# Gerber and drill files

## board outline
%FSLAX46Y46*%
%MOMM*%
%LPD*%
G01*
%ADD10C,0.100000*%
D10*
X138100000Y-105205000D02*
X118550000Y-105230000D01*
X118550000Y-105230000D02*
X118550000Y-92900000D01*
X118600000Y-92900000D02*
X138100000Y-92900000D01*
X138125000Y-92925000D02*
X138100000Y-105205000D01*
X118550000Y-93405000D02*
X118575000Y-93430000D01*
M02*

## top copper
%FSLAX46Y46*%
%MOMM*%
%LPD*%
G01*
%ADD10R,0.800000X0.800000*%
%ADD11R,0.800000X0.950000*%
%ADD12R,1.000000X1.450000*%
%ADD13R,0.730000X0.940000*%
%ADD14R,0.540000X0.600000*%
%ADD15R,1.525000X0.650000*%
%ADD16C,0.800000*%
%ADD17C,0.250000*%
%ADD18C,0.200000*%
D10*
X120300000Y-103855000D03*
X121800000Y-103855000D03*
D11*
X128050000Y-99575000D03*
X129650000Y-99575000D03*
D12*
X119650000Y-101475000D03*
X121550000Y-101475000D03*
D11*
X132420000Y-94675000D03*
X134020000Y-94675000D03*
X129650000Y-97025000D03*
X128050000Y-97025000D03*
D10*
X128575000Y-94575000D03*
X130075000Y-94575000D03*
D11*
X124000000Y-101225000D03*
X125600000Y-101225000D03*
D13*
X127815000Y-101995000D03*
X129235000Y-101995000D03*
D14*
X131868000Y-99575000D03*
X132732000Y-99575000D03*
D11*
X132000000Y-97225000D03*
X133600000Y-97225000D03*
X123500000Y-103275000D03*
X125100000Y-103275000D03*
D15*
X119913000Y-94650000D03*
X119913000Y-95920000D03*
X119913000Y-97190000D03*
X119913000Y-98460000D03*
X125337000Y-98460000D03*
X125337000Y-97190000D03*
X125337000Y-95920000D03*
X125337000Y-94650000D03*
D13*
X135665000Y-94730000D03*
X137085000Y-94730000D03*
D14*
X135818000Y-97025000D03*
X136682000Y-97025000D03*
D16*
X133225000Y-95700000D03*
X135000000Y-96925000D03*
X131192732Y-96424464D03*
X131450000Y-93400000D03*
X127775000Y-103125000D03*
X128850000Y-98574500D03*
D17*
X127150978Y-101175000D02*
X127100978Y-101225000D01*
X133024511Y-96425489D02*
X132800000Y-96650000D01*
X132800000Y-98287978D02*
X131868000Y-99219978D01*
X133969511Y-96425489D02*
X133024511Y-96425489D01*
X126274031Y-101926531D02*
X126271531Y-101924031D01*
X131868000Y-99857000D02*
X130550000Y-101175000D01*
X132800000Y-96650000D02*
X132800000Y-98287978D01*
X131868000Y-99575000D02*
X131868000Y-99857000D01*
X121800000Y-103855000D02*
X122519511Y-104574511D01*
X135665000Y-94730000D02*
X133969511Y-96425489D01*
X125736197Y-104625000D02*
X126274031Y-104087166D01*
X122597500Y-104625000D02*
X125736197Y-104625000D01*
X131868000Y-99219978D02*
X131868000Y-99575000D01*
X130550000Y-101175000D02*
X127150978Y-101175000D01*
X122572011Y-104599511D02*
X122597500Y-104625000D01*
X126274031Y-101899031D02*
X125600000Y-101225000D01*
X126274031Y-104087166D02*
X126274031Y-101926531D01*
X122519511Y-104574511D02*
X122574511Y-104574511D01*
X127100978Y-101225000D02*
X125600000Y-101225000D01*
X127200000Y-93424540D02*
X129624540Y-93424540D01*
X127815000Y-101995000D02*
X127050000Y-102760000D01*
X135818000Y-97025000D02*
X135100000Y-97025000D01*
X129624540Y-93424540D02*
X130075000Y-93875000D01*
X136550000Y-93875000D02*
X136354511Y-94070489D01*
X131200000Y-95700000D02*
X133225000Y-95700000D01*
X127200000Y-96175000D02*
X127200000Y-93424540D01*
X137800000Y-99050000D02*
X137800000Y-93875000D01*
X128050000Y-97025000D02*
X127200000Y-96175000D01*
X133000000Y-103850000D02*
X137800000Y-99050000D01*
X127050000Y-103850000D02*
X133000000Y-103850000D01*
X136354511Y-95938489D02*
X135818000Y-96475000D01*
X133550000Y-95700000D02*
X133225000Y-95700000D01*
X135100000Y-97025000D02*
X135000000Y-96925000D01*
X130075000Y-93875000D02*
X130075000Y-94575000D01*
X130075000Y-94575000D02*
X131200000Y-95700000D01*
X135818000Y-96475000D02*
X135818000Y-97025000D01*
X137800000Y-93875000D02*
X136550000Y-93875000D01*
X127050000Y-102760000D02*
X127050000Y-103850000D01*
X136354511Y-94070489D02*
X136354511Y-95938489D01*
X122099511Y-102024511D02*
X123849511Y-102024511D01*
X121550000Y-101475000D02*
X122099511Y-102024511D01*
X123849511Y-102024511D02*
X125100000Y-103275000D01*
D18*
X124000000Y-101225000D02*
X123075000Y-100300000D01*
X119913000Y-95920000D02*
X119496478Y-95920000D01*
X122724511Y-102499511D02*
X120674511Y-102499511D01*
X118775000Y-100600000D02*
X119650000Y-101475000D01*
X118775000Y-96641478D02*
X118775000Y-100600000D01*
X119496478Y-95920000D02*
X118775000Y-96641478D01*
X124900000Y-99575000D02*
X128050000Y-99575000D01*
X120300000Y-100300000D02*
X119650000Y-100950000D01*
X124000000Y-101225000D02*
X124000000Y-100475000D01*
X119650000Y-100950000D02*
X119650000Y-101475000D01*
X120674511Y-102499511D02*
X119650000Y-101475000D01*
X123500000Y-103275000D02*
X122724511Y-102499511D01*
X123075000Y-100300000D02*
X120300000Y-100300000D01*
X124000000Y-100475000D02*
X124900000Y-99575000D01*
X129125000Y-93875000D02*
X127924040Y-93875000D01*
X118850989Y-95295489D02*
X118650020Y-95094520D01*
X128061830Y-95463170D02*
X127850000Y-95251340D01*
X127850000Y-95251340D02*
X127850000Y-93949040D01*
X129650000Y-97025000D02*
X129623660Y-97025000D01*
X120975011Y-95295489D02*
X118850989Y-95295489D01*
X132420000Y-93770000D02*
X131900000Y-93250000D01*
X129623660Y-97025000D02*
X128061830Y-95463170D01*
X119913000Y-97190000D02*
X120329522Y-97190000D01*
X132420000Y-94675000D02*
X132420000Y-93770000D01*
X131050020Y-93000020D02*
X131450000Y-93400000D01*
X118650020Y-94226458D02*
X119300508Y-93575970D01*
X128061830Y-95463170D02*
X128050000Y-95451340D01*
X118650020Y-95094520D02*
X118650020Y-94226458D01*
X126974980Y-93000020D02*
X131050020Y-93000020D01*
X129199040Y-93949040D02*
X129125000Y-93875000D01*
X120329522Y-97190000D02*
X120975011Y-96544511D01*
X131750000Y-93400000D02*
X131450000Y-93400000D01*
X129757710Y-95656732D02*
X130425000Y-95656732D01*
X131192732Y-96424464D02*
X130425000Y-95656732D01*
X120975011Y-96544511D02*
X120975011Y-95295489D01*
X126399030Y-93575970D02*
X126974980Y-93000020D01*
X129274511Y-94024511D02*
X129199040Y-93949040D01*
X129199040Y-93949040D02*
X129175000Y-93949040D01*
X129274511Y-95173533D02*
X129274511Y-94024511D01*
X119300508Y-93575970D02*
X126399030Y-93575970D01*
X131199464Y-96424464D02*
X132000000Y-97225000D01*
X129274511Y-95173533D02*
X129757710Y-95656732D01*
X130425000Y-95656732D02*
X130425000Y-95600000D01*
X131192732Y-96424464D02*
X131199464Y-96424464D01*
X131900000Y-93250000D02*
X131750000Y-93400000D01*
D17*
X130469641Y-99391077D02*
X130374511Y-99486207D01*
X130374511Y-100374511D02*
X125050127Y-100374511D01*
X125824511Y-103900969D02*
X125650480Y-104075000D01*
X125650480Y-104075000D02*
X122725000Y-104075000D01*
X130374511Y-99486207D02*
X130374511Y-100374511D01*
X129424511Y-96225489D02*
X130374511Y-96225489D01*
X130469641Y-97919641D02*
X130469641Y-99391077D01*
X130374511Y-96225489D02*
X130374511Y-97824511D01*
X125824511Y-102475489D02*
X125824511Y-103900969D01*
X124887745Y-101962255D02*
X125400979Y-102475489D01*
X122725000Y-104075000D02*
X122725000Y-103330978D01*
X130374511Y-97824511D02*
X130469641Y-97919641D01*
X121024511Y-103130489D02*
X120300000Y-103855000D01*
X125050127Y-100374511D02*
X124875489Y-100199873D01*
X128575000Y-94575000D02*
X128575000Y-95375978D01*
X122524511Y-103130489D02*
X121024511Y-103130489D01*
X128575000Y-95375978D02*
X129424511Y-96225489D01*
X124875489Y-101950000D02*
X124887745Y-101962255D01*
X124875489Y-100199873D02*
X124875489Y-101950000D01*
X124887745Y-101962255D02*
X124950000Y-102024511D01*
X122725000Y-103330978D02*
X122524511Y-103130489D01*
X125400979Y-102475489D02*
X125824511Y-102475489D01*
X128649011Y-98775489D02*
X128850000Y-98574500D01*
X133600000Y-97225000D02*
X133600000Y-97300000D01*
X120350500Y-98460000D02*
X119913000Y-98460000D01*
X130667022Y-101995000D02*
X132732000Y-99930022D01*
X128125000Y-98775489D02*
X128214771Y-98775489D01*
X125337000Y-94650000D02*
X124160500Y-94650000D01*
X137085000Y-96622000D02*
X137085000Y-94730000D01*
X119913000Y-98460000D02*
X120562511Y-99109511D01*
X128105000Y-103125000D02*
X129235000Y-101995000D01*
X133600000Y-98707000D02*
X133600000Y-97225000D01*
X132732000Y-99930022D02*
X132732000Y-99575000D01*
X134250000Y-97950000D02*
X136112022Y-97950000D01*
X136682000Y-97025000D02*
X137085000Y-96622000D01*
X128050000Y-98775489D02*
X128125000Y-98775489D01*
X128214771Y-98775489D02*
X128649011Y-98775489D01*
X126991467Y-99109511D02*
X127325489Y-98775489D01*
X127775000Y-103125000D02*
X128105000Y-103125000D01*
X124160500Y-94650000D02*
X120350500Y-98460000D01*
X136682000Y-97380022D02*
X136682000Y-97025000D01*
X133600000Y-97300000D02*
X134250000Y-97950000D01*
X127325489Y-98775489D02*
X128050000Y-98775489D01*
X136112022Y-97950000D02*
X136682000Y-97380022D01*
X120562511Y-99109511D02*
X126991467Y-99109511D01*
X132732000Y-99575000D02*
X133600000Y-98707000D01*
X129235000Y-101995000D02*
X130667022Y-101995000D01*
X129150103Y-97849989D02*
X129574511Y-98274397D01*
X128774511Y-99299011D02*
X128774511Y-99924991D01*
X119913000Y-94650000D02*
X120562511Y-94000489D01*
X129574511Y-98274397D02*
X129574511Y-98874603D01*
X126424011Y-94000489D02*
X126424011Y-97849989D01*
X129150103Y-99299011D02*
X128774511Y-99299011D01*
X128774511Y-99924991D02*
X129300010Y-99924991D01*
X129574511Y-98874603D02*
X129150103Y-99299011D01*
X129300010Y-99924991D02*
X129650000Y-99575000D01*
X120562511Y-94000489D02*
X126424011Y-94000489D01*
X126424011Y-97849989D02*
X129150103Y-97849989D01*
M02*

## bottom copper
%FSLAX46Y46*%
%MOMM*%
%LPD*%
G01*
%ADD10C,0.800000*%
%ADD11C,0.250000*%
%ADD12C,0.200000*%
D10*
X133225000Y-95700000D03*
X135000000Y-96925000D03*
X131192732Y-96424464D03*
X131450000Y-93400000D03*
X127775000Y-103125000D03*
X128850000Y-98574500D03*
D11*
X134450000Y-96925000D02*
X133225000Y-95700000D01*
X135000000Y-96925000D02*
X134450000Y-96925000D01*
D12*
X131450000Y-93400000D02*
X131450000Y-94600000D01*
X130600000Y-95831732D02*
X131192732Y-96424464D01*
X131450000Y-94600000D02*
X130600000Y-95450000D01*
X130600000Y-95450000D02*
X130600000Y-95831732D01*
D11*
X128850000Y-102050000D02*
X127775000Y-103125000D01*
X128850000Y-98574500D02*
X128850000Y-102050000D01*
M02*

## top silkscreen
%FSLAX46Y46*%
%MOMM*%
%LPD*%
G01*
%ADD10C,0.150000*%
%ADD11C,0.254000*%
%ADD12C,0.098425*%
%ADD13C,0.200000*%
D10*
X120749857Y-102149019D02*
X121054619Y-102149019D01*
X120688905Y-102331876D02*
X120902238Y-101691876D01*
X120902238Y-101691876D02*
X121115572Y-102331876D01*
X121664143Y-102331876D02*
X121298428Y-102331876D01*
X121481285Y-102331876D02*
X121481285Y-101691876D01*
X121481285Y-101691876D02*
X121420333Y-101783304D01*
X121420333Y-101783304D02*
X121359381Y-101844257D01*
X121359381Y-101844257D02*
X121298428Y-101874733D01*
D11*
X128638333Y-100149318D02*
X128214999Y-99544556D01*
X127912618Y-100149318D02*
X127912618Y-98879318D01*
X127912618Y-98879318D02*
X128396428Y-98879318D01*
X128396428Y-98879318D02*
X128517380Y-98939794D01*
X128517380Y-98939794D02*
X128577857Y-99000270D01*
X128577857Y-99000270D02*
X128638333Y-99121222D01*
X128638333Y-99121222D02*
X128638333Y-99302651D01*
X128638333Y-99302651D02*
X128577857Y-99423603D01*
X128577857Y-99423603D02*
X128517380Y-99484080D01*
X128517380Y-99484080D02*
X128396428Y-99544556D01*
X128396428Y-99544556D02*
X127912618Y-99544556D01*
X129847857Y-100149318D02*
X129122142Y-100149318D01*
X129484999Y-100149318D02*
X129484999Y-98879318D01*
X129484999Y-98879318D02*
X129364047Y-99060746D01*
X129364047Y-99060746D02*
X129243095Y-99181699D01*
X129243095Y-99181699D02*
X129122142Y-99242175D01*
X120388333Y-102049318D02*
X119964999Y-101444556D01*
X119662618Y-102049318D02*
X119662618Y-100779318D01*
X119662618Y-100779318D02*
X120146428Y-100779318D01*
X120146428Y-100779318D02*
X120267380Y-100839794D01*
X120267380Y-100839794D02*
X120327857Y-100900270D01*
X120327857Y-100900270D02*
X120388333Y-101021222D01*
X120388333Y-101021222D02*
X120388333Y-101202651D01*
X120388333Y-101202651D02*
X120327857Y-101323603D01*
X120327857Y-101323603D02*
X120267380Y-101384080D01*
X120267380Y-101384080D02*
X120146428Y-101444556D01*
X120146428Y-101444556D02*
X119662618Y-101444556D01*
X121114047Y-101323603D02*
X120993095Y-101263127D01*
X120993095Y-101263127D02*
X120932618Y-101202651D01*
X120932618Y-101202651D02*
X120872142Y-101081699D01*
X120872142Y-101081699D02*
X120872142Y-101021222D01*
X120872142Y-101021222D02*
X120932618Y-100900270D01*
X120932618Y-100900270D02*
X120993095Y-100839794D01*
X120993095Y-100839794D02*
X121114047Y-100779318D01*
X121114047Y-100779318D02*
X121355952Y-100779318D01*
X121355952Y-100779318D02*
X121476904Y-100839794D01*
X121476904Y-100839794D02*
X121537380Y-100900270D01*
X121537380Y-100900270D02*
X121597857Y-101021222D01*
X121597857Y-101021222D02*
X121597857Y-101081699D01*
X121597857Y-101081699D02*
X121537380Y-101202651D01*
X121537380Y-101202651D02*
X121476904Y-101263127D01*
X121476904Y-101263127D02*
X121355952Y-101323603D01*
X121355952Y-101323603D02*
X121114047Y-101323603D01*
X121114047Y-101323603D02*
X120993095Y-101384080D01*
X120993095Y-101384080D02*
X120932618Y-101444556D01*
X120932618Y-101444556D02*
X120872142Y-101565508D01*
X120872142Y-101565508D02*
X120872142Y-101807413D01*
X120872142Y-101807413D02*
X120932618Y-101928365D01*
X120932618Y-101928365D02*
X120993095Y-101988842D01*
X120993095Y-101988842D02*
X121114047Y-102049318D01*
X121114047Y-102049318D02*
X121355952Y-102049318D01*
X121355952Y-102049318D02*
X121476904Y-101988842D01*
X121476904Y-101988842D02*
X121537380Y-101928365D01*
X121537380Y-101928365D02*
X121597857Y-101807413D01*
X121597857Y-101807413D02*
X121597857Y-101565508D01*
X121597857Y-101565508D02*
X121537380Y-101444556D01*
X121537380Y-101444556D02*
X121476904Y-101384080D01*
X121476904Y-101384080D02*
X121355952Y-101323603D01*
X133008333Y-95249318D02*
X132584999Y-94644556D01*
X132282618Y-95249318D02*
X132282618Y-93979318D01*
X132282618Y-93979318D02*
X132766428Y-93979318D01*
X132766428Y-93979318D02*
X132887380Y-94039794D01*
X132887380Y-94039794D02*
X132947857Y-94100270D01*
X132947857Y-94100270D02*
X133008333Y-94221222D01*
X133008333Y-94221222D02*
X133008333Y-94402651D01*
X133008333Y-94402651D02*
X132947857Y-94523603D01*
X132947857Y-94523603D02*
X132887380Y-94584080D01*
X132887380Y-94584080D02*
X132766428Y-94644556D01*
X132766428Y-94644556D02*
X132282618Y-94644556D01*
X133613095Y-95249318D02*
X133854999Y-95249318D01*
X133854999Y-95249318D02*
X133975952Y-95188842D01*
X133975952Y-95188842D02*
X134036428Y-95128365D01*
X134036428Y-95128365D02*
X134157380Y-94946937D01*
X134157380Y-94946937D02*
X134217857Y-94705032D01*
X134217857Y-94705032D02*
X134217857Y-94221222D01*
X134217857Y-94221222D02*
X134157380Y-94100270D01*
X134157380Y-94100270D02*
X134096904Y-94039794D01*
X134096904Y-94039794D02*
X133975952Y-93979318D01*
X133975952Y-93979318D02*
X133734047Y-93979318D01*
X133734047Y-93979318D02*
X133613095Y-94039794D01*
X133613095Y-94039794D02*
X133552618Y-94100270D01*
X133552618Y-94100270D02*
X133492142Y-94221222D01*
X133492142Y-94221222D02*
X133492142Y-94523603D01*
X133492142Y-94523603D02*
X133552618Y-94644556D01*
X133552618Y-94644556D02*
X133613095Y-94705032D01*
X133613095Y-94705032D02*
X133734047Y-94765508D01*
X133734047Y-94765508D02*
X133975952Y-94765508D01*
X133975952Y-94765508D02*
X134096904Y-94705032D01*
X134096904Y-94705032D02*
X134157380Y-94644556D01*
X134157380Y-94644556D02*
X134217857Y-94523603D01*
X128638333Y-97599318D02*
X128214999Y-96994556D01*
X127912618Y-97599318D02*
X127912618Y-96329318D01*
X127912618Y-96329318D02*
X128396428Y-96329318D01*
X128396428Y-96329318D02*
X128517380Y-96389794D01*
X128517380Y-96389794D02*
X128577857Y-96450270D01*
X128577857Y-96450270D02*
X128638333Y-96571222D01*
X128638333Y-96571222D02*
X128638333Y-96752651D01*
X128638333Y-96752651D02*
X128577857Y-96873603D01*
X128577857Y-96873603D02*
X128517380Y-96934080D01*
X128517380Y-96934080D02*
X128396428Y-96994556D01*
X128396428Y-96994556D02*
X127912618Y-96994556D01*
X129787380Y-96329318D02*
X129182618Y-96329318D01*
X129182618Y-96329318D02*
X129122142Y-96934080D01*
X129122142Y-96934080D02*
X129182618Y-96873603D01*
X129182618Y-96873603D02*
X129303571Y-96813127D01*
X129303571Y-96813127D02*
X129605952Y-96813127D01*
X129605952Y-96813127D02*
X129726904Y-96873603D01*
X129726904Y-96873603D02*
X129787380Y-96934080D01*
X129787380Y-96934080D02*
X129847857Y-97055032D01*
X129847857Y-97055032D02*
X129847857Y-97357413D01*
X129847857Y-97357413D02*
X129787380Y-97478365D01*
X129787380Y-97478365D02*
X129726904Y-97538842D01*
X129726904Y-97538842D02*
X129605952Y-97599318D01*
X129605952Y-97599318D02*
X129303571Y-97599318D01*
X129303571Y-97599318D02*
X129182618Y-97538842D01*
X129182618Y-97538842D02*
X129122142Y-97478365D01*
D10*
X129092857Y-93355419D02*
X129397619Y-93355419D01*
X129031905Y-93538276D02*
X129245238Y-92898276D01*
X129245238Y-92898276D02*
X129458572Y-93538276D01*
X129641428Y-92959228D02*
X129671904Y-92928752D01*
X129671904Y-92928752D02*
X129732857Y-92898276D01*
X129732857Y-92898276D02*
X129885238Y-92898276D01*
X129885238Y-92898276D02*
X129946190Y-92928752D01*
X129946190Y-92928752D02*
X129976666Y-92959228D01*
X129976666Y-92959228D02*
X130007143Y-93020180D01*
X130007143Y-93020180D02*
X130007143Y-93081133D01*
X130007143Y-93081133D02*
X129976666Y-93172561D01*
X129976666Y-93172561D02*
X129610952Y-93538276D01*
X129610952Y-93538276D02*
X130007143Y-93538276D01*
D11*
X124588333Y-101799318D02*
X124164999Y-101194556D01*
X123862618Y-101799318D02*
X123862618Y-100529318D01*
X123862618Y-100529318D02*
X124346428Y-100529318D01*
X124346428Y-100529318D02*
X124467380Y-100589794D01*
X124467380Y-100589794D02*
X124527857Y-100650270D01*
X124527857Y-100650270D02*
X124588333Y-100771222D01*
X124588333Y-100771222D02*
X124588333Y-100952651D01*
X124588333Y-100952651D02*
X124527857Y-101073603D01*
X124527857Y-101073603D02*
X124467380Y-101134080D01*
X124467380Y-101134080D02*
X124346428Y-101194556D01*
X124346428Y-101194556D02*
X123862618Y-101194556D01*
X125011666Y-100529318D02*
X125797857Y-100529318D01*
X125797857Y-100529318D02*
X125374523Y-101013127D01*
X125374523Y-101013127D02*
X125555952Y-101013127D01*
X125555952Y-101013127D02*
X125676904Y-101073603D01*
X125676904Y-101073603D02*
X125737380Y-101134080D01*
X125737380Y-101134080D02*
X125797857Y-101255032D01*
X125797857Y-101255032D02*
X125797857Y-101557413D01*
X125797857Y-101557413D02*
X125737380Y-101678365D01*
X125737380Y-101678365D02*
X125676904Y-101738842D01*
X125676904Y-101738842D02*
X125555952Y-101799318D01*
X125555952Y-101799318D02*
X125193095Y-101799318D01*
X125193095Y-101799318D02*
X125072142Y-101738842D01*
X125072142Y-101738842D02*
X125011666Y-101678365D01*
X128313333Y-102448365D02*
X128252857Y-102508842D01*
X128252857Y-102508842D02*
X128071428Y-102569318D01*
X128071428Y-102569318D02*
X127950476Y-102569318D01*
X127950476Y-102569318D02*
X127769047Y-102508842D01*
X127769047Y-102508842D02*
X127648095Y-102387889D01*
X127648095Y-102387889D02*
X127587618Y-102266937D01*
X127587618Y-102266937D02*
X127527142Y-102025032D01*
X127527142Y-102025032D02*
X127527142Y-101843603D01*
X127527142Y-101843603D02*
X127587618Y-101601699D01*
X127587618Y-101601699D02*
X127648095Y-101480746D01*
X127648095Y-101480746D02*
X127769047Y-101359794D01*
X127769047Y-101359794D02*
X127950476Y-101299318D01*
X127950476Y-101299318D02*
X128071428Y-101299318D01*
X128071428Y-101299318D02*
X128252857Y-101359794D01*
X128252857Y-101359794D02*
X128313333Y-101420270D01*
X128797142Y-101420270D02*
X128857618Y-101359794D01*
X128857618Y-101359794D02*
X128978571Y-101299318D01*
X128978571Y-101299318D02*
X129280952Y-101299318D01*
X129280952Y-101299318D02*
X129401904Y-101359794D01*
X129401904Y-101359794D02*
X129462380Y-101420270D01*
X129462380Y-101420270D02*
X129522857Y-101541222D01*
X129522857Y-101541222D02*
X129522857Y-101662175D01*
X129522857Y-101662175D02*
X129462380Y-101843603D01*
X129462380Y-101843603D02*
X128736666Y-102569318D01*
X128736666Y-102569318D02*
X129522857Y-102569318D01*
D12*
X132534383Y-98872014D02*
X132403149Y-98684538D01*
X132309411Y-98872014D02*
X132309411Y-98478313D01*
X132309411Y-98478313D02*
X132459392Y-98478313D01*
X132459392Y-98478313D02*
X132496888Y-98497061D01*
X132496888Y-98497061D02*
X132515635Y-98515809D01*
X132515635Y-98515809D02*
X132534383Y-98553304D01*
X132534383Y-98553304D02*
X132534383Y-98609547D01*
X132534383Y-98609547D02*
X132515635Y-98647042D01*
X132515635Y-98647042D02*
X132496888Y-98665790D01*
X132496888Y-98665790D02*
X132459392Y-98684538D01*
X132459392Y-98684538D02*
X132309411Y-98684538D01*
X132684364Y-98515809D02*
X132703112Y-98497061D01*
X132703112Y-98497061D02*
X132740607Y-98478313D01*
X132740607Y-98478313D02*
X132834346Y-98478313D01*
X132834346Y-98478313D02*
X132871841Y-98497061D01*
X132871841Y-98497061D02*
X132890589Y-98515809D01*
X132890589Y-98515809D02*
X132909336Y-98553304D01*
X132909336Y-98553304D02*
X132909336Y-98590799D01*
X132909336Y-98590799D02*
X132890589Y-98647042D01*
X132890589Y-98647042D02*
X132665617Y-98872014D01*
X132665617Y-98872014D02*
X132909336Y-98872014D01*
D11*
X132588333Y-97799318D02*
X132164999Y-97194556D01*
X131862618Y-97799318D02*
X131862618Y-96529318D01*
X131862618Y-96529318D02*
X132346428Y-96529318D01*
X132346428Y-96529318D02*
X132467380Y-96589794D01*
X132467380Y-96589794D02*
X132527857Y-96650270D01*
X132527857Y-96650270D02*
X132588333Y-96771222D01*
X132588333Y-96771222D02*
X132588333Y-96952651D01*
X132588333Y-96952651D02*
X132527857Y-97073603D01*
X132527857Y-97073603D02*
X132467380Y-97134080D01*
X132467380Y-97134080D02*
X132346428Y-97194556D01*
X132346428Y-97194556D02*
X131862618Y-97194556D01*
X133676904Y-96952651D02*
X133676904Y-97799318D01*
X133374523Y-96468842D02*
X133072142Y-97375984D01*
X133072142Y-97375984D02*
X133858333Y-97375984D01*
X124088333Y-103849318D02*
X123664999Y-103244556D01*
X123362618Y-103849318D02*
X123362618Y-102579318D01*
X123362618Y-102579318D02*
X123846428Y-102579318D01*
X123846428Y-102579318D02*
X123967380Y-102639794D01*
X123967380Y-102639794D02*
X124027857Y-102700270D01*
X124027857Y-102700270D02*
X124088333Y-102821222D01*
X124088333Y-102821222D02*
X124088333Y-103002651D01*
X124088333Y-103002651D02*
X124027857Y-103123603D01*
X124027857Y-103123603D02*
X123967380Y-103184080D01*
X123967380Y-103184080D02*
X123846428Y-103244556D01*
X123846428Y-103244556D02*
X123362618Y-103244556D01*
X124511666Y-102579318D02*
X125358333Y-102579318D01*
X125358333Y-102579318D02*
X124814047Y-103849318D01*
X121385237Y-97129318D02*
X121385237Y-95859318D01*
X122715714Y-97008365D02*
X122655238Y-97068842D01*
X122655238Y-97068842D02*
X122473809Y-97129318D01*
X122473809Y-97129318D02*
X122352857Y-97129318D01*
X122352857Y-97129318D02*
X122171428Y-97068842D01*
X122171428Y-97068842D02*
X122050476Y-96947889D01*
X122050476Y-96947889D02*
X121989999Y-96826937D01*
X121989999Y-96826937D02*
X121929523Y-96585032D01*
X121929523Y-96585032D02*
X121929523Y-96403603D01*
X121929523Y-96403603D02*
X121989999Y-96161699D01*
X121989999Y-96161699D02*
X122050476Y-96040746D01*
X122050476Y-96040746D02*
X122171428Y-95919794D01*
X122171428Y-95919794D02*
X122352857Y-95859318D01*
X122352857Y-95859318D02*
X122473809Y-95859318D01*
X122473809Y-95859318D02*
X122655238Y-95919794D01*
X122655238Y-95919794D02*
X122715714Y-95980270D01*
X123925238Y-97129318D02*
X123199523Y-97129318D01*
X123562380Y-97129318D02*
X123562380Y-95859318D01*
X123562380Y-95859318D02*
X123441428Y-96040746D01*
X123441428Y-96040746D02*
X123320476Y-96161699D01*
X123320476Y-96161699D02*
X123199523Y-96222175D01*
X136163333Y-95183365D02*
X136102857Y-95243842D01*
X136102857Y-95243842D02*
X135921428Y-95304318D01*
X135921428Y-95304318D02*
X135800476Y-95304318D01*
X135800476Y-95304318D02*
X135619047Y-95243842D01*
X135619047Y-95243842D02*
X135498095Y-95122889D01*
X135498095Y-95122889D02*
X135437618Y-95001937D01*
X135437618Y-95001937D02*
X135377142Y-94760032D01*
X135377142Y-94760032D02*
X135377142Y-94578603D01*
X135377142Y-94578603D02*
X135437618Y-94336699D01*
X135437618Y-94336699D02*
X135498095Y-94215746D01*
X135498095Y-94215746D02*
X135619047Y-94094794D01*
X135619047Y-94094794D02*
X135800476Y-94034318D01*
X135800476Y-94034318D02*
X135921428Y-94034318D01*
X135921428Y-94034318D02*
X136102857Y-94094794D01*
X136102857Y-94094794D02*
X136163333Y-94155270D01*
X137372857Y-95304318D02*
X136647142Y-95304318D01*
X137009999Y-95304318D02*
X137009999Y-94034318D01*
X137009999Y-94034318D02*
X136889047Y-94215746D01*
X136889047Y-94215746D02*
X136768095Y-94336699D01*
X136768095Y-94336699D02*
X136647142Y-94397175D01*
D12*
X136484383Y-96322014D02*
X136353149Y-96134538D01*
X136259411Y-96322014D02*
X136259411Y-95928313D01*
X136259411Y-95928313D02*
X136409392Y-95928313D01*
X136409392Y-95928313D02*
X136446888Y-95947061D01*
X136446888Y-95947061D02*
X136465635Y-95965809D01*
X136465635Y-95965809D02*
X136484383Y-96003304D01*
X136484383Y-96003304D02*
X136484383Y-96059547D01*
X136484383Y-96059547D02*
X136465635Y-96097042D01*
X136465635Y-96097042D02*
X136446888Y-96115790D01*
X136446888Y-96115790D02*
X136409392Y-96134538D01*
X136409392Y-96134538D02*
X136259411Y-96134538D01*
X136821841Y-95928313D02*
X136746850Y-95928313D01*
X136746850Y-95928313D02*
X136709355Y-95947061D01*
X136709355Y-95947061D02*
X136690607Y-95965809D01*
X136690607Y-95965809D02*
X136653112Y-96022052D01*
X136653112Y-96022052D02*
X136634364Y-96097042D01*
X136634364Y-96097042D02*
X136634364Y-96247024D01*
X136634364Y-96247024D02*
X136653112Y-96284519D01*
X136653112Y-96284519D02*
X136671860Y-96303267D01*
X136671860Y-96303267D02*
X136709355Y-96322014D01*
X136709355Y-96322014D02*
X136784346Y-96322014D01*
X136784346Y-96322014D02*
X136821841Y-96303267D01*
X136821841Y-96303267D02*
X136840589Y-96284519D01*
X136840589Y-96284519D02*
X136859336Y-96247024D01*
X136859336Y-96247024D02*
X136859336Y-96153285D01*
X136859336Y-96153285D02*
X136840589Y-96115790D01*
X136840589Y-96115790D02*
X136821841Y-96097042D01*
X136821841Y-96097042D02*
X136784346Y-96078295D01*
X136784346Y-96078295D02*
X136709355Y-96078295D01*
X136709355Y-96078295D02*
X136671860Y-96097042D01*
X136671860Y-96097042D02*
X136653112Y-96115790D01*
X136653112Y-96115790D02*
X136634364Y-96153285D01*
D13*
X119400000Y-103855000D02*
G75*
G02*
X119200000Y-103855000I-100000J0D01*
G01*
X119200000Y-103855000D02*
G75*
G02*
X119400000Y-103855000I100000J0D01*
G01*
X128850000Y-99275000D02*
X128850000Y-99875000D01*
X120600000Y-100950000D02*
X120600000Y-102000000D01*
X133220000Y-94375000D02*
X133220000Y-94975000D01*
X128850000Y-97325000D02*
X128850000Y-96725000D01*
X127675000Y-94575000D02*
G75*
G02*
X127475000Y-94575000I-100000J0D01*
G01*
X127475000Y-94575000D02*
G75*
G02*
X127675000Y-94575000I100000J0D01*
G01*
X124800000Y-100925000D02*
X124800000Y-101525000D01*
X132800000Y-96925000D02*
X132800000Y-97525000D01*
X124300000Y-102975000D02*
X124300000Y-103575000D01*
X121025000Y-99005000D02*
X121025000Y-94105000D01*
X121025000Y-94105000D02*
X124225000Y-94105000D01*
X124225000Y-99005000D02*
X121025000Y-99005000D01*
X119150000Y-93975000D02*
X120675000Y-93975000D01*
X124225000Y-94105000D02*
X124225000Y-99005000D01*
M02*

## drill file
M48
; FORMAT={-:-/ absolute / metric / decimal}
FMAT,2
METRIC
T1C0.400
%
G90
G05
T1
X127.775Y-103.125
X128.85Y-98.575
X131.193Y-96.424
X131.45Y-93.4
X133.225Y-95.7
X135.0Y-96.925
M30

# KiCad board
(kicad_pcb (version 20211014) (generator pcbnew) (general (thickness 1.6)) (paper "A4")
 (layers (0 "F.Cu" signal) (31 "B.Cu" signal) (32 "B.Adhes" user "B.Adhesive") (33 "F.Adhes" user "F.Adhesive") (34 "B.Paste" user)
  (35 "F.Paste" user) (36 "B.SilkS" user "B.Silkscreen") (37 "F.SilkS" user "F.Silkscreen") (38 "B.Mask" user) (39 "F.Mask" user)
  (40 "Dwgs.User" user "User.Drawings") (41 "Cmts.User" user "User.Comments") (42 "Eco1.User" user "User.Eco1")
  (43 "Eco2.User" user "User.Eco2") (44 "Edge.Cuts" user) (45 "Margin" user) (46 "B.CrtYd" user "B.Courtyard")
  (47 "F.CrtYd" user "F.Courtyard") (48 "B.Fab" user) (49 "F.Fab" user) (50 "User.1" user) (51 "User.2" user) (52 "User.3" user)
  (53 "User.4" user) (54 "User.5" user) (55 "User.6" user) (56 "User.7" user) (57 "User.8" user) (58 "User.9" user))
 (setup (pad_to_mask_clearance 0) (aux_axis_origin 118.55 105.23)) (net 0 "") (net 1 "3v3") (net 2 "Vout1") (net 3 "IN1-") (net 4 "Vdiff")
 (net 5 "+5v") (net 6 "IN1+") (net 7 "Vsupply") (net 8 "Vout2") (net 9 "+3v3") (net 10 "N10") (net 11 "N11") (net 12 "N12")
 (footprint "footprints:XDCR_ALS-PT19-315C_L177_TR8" (layer "F.Cu") (at 121.05 103.855)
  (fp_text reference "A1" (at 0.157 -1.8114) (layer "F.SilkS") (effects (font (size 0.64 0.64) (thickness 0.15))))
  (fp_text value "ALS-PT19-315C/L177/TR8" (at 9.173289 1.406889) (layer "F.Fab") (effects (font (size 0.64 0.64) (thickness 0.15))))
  (fp_circle (center -1.75 0) (end -1.65 0) (layer "F.SilkS") (width 0.2) (fill none))
  (pad "1" smd rect locked (at -0.75 0) (size 0.8 0.8) (layers "F.Cu" "F.Paste" "F.Mask") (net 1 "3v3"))
  (pad "2" smd rect locked (at 0.75 0) (size 0.8 0.8) (layers "F.Cu" "F.Paste" "F.Mask") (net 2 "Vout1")))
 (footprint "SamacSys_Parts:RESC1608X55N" (layer "F.Cu") (at 128.85 99.575)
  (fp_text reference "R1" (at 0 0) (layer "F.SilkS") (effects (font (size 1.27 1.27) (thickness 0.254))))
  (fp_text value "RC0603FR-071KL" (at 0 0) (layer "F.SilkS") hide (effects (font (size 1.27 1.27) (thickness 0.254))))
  (fp_line (start 0 -0.3) (end 0 0.3) (layer "F.SilkS") (width 0.2))
  (pad "1" smd rect locked (at -0.8 0) (size 0.8 0.95) (layers "F.Cu" "F.Paste" "F.Mask") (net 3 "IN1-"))
  (pad "2" smd rect locked (at 0.8 0) (size 0.8 0.95) (layers "F.Cu" "F.Paste" "F.Mask") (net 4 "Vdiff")))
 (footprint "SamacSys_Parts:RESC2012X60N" (layer "F.Cu") (at 120.6 101.475)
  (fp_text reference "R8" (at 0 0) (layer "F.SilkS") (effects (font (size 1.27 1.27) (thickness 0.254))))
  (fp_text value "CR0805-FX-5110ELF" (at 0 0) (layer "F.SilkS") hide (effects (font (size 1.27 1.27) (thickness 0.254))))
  (fp_line (start 0 -0.525) (end 0 0.525) (layer "F.SilkS") (width 0.2))
  (pad "1" smd rect locked (at -0.95 0) (size 1 1.45) (layers "F.Cu" "F.Paste" "F.Mask") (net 3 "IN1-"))
  (pad "2" smd rect locked (at 0.95 0) (size 1 1.45) (layers "F.Cu" "F.Paste" "F.Mask") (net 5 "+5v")))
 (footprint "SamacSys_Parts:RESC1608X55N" (layer "F.Cu") (at 133.22 94.675)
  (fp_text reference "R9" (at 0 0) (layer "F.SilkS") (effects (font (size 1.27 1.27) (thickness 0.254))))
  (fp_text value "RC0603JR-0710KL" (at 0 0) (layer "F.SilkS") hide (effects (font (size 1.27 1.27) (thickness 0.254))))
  (fp_line (start 0 -0.3) (end 0 0.3) (layer "F.SilkS") (width 0.2))
  (pad "1" smd rect locked (at -0.8 0) (size 0.8 0.95) (layers "F.Cu" "F.Paste" "F.Mask") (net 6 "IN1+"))
  (pad "2" smd rect locked (at 0.8 0) (size 0.8 0.95) (layers "F.Cu" "F.Paste" "F.Mask") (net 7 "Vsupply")))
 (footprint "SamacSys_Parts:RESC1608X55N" (layer "F.Cu") (at 128.85 97.025 180)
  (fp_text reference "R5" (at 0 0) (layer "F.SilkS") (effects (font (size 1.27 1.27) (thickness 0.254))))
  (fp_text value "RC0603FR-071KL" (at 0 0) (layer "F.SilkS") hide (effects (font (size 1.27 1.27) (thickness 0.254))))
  (fp_line (start 0 -0.3) (end 0 0.3) (layer "F.SilkS") (width 0.2))
  (pad "1" smd rect locked (at -0.8 0 180) (size 0.8 0.95) (layers "F.Cu" "F.Paste" "F.Mask") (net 6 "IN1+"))
  (pad "2" smd rect locked (at 0.8 0 180) (size 0.8 0.95) (layers "F.Cu" "F.Paste" "F.Mask") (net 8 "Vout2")))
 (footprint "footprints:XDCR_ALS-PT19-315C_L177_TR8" (layer "F.Cu") (at 129.325 94.575)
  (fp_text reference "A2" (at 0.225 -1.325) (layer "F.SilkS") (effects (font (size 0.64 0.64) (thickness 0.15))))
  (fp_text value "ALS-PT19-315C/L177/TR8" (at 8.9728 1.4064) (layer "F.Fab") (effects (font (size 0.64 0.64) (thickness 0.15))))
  (fp_circle (center -1.75 0) (end -1.65 0) (layer "F.SilkS") (width 0.2) (fill none))
  (pad "1" smd rect locked (at -0.75 0) (size 0.8 0.8) (layers "F.Cu" "F.Paste" "F.Mask") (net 1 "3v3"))
  (pad "2" smd rect locked (at 0.75 0) (size 0.8 0.8) (layers "F.Cu" "F.Paste" "F.Mask") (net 8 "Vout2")))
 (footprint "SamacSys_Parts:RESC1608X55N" (layer "F.Cu") (at 124.8 101.225)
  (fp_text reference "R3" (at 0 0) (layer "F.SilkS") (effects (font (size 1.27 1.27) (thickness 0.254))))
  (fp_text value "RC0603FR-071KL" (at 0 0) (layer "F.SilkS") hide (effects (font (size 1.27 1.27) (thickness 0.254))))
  (fp_line (start 0 -0.3) (end 0 0.3) (layer "F.SilkS") (width 0.2))
  (pad "1" smd rect locked (at -0.8 0) (size 0.8 0.95) (layers "F.Cu" "F.Paste" "F.Mask") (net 3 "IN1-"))
  (pad "2" smd rect locked (at 0.8 0) (size 0.8 0.95) (layers "F.Cu" "F.Paste" "F.Mask") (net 2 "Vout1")))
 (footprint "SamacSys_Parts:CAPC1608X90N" (layer "F.Cu") (at 128.525 101.995)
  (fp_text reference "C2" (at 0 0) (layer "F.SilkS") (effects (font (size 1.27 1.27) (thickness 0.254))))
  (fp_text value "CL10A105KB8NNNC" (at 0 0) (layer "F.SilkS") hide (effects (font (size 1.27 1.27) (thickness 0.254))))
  (pad "1" smd rect locked (at -0.71 0) (size 0.73 0.94) (layers "F.Cu" "F.Paste" "F.Mask") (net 8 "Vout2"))
  (pad "2" smd rect locked (at 0.71 0) (size 0.73 0.94) (layers "F.Cu" "F.Paste" "F.Mask") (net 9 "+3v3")))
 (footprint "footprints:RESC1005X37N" (layer "F.Cu") (at 132.3 99.575)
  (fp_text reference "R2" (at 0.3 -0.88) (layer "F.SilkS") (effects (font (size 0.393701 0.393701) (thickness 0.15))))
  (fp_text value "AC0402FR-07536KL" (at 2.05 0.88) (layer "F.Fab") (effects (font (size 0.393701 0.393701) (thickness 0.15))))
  (pad "1" smd rect locked (at -0.432 0) (size 0.54 0.6) (layers "F.Cu" "F.Paste" "F.Mask") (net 2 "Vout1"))
  (pad "2" smd rect locked (at 0.432 0) (size 0.54 0.6) (layers "F.Cu" "F.Paste" "F.Mask") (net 9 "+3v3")))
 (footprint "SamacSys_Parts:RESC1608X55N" (layer "F.Cu") (at 132.8 97.225)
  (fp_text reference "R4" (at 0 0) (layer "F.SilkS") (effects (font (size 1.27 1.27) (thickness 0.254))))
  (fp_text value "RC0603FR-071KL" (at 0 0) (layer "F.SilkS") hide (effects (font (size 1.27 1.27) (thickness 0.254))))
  (fp_line (start 0 -0.3) (end 0 0.3) (layer "F.SilkS") (width 0.2))
  (pad "1" smd rect locked (at -0.8 0) (size 0.8 0.95) (layers "F.Cu" "F.Paste" "F.Mask") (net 6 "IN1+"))
  (pad "2" smd rect locked (at 0.8 0) (size 0.8 0.95) (layers "F.Cu" "F.Paste" "F.Mask") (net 9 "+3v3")))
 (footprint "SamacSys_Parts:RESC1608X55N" (layer "F.Cu") (at 124.3 103.275)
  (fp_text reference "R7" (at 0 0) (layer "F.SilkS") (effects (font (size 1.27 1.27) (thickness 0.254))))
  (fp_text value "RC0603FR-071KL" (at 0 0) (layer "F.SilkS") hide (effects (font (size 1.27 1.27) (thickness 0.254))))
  (fp_line (start 0 -0.3) (end 0 0.3) (layer "F.SilkS") (width 0.2))
  (pad "1" smd rect locked (at -0.8 0) (size 0.8 0.95) (layers "F.Cu" "F.Paste" "F.Mask") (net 3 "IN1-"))
  (pad "2" smd rect locked (at 0.8 0) (size 0.8 0.95) (layers "F.Cu" "F.Paste" "F.Mask") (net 5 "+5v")))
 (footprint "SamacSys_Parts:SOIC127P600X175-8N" (layer "F.Cu") (at 122.625 96.555)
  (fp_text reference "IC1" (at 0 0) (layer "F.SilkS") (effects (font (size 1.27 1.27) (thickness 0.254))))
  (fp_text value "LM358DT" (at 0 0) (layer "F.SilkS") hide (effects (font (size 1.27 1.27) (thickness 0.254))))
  (fp_line (start -1.6 2.45) (end -1.6 -2.45) (layer "F.SilkS") (width 0.2))
  (fp_line (start -1.6 -2.45) (end 1.6 -2.45) (layer "F.SilkS") (width 0.2))
  (fp_line (start 1.6 2.45) (end -1.6 2.45) (layer "F.SilkS") (width 0.2))
  (fp_line (start -3.475 -2.58) (end -1.95 -2.58) (layer "F.SilkS") (width 0.2))
  (fp_line (start 1.6 -2.45) (end 1.6 2.45) (layer "F.SilkS") (width 0.2))
  (pad "1" smd rect locked (at -2.712 -1.905 90) (size 0.65 1.525) (layers "F.Cu" "F.Paste" "F.Mask") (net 4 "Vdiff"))
  (pad "2" smd rect locked (at -2.712 -0.635 90) (size 0.65 1.525) (layers "F.Cu" "F.Paste" "F.Mask") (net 3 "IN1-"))
  (pad "3" smd rect locked (at -2.712 0.635 90) (size 0.65 1.525) (layers "F.Cu" "F.Paste" "F.Mask") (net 6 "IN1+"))
  (pad "4" smd rect locked (at -2.712 1.905 90) (size 0.65 1.525) (layers "F.Cu" "F.Paste" "F.Mask") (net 9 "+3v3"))
  (pad "5" smd rect locked (at 2.712 1.905 90) (size 0.65 1.525) (layers "F.Cu" "F.Paste" "F.Mask") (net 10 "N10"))
  (pad "6" smd rect locked (at 2.712 0.635 90) (size 0.65 1.525) (layers "F.Cu" "F.Paste" "F.Mask") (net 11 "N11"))
  (pad "7" smd rect locked (at 2.712 -0.635 90) (size 0.65 1.525) (layers "F.Cu" "F.Paste" "F.Mask") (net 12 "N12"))
  (pad "8" smd rect locked (at 2.712 -1.905 90) (size 0.65 1.525) (layers "F.Cu" "F.Paste" "F.Mask") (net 9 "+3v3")))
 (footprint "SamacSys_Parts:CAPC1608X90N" (layer "F.Cu") (at 136.375 94.73)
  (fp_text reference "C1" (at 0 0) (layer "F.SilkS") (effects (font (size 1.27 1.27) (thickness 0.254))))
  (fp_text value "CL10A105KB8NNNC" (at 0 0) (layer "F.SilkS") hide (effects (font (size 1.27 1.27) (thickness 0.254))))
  (pad "1" smd rect locked (at -0.71 0) (size 0.73 0.94) (layers "F.Cu" "F.Paste" "F.Mask") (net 2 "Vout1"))
  (pad "2" smd rect locked (at 0.71 0) (size 0.73 0.94) (layers "F.Cu" "F.Paste" "F.Mask") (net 9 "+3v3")))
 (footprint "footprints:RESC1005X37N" (layer "F.Cu") (at 136.25 97.025)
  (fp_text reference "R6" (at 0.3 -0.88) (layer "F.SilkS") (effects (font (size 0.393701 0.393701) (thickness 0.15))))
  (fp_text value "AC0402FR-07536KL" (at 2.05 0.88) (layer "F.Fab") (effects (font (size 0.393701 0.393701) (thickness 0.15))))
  (pad "1" smd rect locked (at -0.432 0) (size 0.54 0.6) (layers "F.Cu" "F.Paste" "F.Mask") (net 8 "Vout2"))
  (pad "2" smd rect locked (at 0.432 0) (size 0.54 0.6) (layers "F.Cu" "F.Paste" "F.Mask") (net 9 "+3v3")))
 (gr_line (start 138.1 105.205) (end 118.55 105.23) (layer "Edge.Cuts") (width 0.1))
 (gr_line (start 118.55 105.23) (end 118.55 92.9) (layer "Edge.Cuts") (width 0.1))
 (gr_line (start 118.6 92.9) (end 138.1 92.9) (layer "Edge.Cuts") (width 0.1))
 (gr_line (start 138.125 92.925) (end 138.1 105.205) (layer "Edge.Cuts") (width 0.1))
 (gr_line (start 118.55 93.405) (end 118.575 93.43) (layer "Edge.Cuts") (width 0.1))
 (segment (start 127.150978 101.175) (end 127.100978 101.225) (width 0.25) (layer "F.Cu") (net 2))
 (segment (start 133.024511 96.425489) (end 132.8 96.65) (width 0.25) (layer "F.Cu") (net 2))
 (segment (start 132.8 98.287978) (end 131.868 99.219978) (width 0.25) (layer "F.Cu") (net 2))
 (segment (start 133.969511 96.425489) (end 133.024511 96.425489) (width 0.25) (layer "F.Cu") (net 2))
 (segment (start 126.274031 101.926531) (end 126.271531 101.924031) (width 0.25) (layer "F.Cu") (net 2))
 (segment (start 131.868 99.857) (end 130.55 101.175) (width 0.25) (layer "F.Cu") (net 2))
 (segment (start 132.8 96.65) (end 132.8 98.287978) (width 0.25) (layer "F.Cu") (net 2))
 (segment (start 131.868 99.575) (end 131.868 99.857) (width 0.25) (layer "F.Cu") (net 2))
 (segment (start 121.8 103.855) (end 122.519511 104.574511) (width 0.25) (layer "F.Cu") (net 2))
 (segment (start 135.665 94.73) (end 133.969511 96.425489) (width 0.25) (layer "F.Cu") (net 2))
 (segment (start 125.736197 104.625) (end 126.274031 104.087166) (width 0.25) (layer "F.Cu") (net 2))
 (segment (start 122.5975 104.625) (end 125.736197 104.625) (width 0.25) (layer "F.Cu") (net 2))
 (segment (start 131.868 99.219978) (end 131.868 99.575) (width 0.25) (layer "F.Cu") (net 2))
 (segment (start 130.55 101.175) (end 127.150978 101.175) (width 0.25) (layer "F.Cu") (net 2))
 (segment (start 122.572011 104.599511) (end 122.5975 104.625) (width 0.25) (layer "F.Cu") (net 2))
 (segment (start 126.274031 101.899031) (end 125.6 101.225) (width 0.25) (layer "F.Cu") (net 2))
 (segment (start 126.274031 104.087166) (end 126.274031 101.926531) (width 0.25) (layer "F.Cu") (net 2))
 (segment (start 122.519511 104.574511) (end 122.574511 104.574511) (width 0.25) (layer "F.Cu") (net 2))
 (segment (start 127.100978 101.225) (end 125.6 101.225) (width 0.25) (layer "F.Cu") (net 2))
 (segment (start 127.2 93.42454) (end 129.62454 93.42454) (width 0.25) (layer "F.Cu") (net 8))
 (segment (start 127.815 101.995) (end 127.05 102.76) (width 0.25) (layer "F.Cu") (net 8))
 (segment (start 135.818 97.025) (end 135.1 97.025) (width 0.25) (layer "F.Cu") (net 8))
 (segment (start 129.62454 93.42454) (end 130.075 93.875) (width 0.25) (layer "F.Cu") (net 8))
 (segment (start 136.55 93.875) (end 136.354511 94.070489) (width 0.25) (layer "F.Cu") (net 8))
 (segment (start 131.2 95.7) (end 133.225 95.7) (width 0.25) (layer "F.Cu") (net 8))
 (segment (start 127.2 96.175) (end 127.2 93.42454) (width 0.25) (layer "F.Cu") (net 8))
 (segment (start 137.8 99.05) (end 137.8 93.875) (width 0.25) (layer "F.Cu") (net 8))
 (segment (start 128.05 97.025) (end 127.2 96.175) (width 0.25) (layer "F.Cu") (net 8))
 (segment (start 133 103.85) (end 137.8 99.05) (width 0.25) (layer "F.Cu") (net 8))
 (segment (start 127.05 103.85) (end 133 103.85) (width 0.25) (layer "F.Cu") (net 8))
 (segment (start 136.354511 95.938489) (end 135.818 96.475) (width 0.25) (layer "F.Cu") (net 8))
 (segment (start 133.55 95.7) (end 133.225 95.7) (width 0.25) (layer "F.Cu") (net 8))
 (segment (start 135.1 97.025) (end 135 96.925) (width 0.25) (layer "F.Cu") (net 8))
 (segment (start 130.075 93.875) (end 130.075 94.575) (width 0.25) (layer "F.Cu") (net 8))
 (segment (start 130.075 94.575) (end 131.2 95.7) (width 0.25) (layer "F.Cu") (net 8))
 (segment (start 135.818 96.475) (end 135.818 97.025) (width 0.25) (layer "F.Cu") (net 8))
 (segment (start 137.8 93.875) (end 136.55 93.875) (width 0.25) (layer "F.Cu") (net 8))
 (segment (start 127.05 102.76) (end 127.05 103.85) (width 0.25) (layer "F.Cu") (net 8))
 (segment (start 136.354511 94.070489) (end 136.354511 95.938489) (width 0.25) (layer "F.Cu") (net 8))
 (via (at 133.225 95.7) (size 0.8) (drill 0.4) (layers "F.Cu" "B.Cu") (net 8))
 (via (at 135 96.925) (size 0.8) (drill 0.4) (layers "F.Cu" "B.Cu") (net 8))
 (segment (start 134.45 96.925) (end 133.225 95.7) (width 0.25) (layer "B.Cu") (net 8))
 (segment (start 135 96.925) (end 134.45 96.925) (width 0.25) (layer "B.Cu") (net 8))
 (segment (start 122.099511 102.024511) (end 123.849511 102.024511) (width 0.25) (layer "F.Cu") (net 5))
 (segment (start 121.55 101.475) (end 122.099511 102.024511) (width 0.25) (layer "F.Cu") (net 5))
 (segment (start 123.849511 102.024511) (end 125.1 103.275) (width 0.25) (layer "F.Cu") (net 5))
 (segment (start 124 101.225) (end 123.075 100.3) (width 0.2) (layer "F.Cu") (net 3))
 (segment (start 119.913 95.92) (end 119.496478 95.92) (width 0.2) (layer "F.Cu") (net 3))
 (segment (start 122.724511 102.499511) (end 120.674511 102.499511) (width 0.2) (layer "F.Cu") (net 3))
 (segment (start 118.775 100.6) (end 119.65 101.475) (width 0.2) (layer "F.Cu") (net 3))
 (segment (start 118.775 96.641478) (end 118.775 100.6) (width 0.2) (layer "F.Cu") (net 3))
 (segment (start 119.496478 95.92) (end 118.775 96.641478) (width 0.2) (layer "F.Cu") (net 3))
 (segment (start 124.9 99.575) (end 128.05 99.575) (width 0.2) (layer "F.Cu") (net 3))
 (segment (start 120.3 100.3) (end 119.65 100.95) (width 0.2) (layer "F.Cu") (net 3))
 (segment (start 124 101.225) (end 124 100.475) (width 0.2) (layer "F.Cu") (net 3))
 (segment (start 119.65 100.95) (end 119.65 101.475) (width 0.2) (layer "F.Cu") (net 3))
 (segment (start 120.674511 102.499511) (end 119.65 101.475) (width 0.2) (layer "F.Cu") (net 3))
 (segment (start 123.5 103.275) (end 122.724511 102.499511) (width 0.2) (layer "F.Cu") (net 3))
 (segment (start 123.075 100.3) (end 120.3 100.3) (width 0.2) (layer "F.Cu") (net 3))
 (segment (start 124 100.475) (end 124.9 99.575) (width 0.2) (layer "F.Cu") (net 3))
 (segment (start 129.125 93.875) (end 127.92404 93.875) (width 0.2) (layer "F.Cu") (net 6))
 (segment (start 118.850989 95.295489) (end 118.65002 95.09452) (width 0.2) (layer "F.Cu") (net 6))
 (segment (start 128.06183 95.46317) (end 127.85 95.25134) (width 0.2) (layer "F.Cu") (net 6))
 (segment (start 127.85 95.25134) (end 127.85 93.94904) (width 0.2) (layer "F.Cu") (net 6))
 (segment (start 129.65 97.025) (end 129.62366 97.025) (width 0.2) (layer "F.Cu") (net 6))
 (segment (start 120.975011 95.295489) (end 118.850989 95.295489) (width 0.2) (layer "F.Cu") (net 6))
 (segment (start 132.42 93.77) (end 131.9 93.25) (width 0.2) (layer "F.Cu") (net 6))
 (segment (start 129.62366 97.025) (end 128.06183 95.46317) (width 0.2) (layer "F.Cu") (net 6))
 (segment (start 119.913 97.19) (end 120.329522 97.19) (width 0.2) (layer "F.Cu") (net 6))
 (segment (start 132.42 94.675) (end 132.42 93.77) (width 0.2) (layer "F.Cu") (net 6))
 (segment (start 131.05002 93.00002) (end 131.45 93.4) (width 0.2) (layer "F.Cu") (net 6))
 (segment (start 118.65002 94.226458) (end 119.300508 93.57597) (width 0.2) (layer "F.Cu") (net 6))
 (segment (start 128.06183 95.46317) (end 128.05 95.45134) (width 0.2) (layer "F.Cu") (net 6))
 (segment (start 118.65002 95.09452) (end 118.65002 94.226458) (width 0.2) (layer "F.Cu") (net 6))
 (segment (start 126.97498 93.00002) (end 131.05002 93.00002) (width 0.2) (layer "F.Cu") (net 6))
 (segment (start 129.19904 93.94904) (end 129.125 93.875) (width 0.2) (layer "F.Cu") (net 6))
 (segment (start 120.329522 97.19) (end 120.975011 96.544511) (width 0.2) (layer "F.Cu") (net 6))
 (segment (start 131.75 93.4) (end 131.45 93.4) (width 0.2) (layer "F.Cu") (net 6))
 (segment (start 129.75771 95.656732) (end 130.425 95.656732) (width 0.2) (layer "F.Cu") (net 6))
 (segment (start 131.192732 96.424464) (end 130.425 95.656732) (width 0.2) (layer "F.Cu") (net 6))
 (segment (start 120.975011 96.544511) (end 120.975011 95.295489) (width 0.2) (layer "F.Cu") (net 6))
 (segment (start 126.39903 93.57597) (end 126.97498 93.00002) (width 0.2) (layer "F.Cu") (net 6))
 (segment (start 129.274511 94.024511) (end 129.19904 93.94904) (width 0.2) (layer "F.Cu") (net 6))
 (segment (start 129.19904 93.94904) (end 129.175 93.94904) (width 0.2) (layer "F.Cu") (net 6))
 (segment (start 129.274511 95.173533) (end 129.274511 94.024511) (width 0.2) (layer "F.Cu") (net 6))
 (segment (start 119.300508 93.57597) (end 126.39903 93.57597) (width 0.2) (layer "F.Cu") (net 6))
 (segment (start 131.199464 96.424464) (end 132 97.225) (width 0.2) (layer "F.Cu") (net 6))
 (segment (start 129.274511 95.173533) (end 129.75771 95.656732) (width 0.2) (layer "F.Cu") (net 6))
 (segment (start 130.425 95.656732) (end 130.425 95.6) (width 0.2) (layer "F.Cu") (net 6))
 (segment (start 131.192732 96.424464) (end 131.199464 96.424464) (width 0.2) (layer "F.Cu") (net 6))
 (segment (start 131.9 93.25) (end 131.75 93.4) (width 0.2) (layer "F.Cu") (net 6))
 (via (at 131.192732 96.424464) (size 0.8) (drill 0.4) (layers "F.Cu" "B.Cu") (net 6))
 (via (at 131.45 93.4) (size 0.8) (drill 0.4) (layers "F.Cu" "B.Cu") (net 6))
 (segment (start 131.45 93.4) (end 131.45 94.6) (width 0.2) (layer "B.Cu") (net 6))
 (segment (start 130.6 95.831732) (end 131.192732 96.424464) (width 0.2) (layer "B.Cu") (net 6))
 (segment (start 131.45 94.6) (end 130.6 95.45) (width 0.2) (layer "B.Cu") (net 6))
 (segment (start 130.6 95.45) (end 130.6 95.831732) (width 0.2) (layer "B.Cu") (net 6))
 (segment (start 130.469641 99.391077) (end 130.374511 99.486207) (width 0.25) (layer "F.Cu") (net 1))
 (segment (start 130.374511 100.374511) (end 125.050127 100.374511) (width 0.25) (layer "F.Cu") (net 1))
 (segment (start 125.824511 103.900969) (end 125.65048 104.075) (width 0.25) (layer "F.Cu") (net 1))
 (segment (start 125.65048 104.075) (end 122.725 104.075) (width 0.25) (layer "F.Cu") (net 1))
 (segment (start 130.374511 99.486207) (end 130.374511 100.374511) (width 0.25) (layer "F.Cu") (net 1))
 (segment (start 129.424511 96.225489) (end 130.374511 96.225489) (width 0.25) (layer "F.Cu") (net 1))
 (segment (start 130.469641 97.919641) (end 130.469641 99.391077) (width 0.25) (layer "F.Cu") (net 1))
 (segment (start 130.374511 96.225489) (end 130.374511 97.824511) (width 0.25) (layer "F.Cu") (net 1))
 (segment (start 125.824511 102.475489) (end 125.824511 103.900969) (width 0.25) (layer "F.Cu") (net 1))
 (segment (start 124.887745 101.962255) (end 125.400979 102.475489) (width 0.25) (layer "F.Cu") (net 1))
 (segment (start 122.725 104.075) (end 122.725 103.330978) (width 0.25) (layer "F.Cu") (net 1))
 (segment (start 130.374511 97.824511) (end 130.469641 97.919641) (width 0.25) (layer "F.Cu") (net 1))
 (segment (start 121.024511 103.130489) (end 120.3 103.855) (width 0.25) (layer "F.Cu") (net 1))
 (segment (start 125.050127 100.374511) (end 124.875489 100.199873) (width 0.25) (layer "F.Cu") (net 1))
 (segment (start 128.575 94.575) (end 128.575 95.375978) (width 0.25) (layer "F.Cu") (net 1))
 (segment (start 122.524511 103.130489) (end 121.024511 103.130489) (width 0.25) (layer "F.Cu") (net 1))
 (segment (start 128.575 95.375978) (end 129.424511 96.225489) (width 0.25) (layer "F.Cu") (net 1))
 (segment (start 124.875489 101.95) (end 124.887745 101.962255) (width 0.25) (layer "F.Cu") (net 1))
 (segment (start 124.875489 100.199873) (end 124.875489 101.95) (width 0.25) (layer "F.Cu") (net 1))
 (segment (start 124.887745 101.962255) (end 124.95 102.024511) (width 0.25) (layer "F.Cu") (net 1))
 (segment (start 122.725 103.330978) (end 122.524511 103.130489) (width 0.25) (layer "F.Cu") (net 1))
 (segment (start 125.400979 102.475489) (end 125.824511 102.475489) (width 0.25) (layer "F.Cu") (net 1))
 (segment (start 128.649011 98.775489) (end 128.85 98.5745) (width 0.25) (layer "F.Cu") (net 9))
 (segment (start 133.6 97.225) (end 133.6 97.3) (width 0.25) (layer "F.Cu") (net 9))
 (segment (start 120.3505 98.46) (end 119.913 98.46) (width 0.25) (layer "F.Cu") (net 9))
 (segment (start 130.667022 101.995) (end 132.732 99.930022) (width 0.25) (layer "F.Cu") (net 9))
 (segment (start 128.125 98.775489) (end 128.214771 98.775489) (width 0.25) (layer "F.Cu") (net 9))
 (segment (start 125.337 94.65) (end 124.1605 94.65) (width 0.25) (layer "F.Cu") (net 9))
 (segment (start 137.085 96.622) (end 137.085 94.73) (width 0.25) (layer "F.Cu") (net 9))
 (segment (start 119.913 98.46) (end 120.562511 99.109511) (width 0.25) (layer "F.Cu") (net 9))
 (segment (start 128.105 103.125) (end 129.235 101.995) (width 0.25) (layer "F.Cu") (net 9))
 (segment (start 133.6 98.707) (end 133.6 97.225) (width 0.25) (layer "F.Cu") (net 9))
 (segment (start 132.732 99.930022) (end 132.732 99.575) (width 0.25) (layer "F.Cu") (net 9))
 (segment (start 134.25 97.95) (end 136.112022 97.95) (width 0.25) (layer "F.Cu") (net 9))
 (segment (start 136.682 97.025) (end 137.085 96.622) (width 0.25) (layer "F.Cu") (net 9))
 (segment (start 128.05 98.775489) (end 128.125 98.775489) (width 0.25) (layer "F.Cu") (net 9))
 (segment (start 128.214771 98.775489) (end 128.649011 98.775489) (width 0.25) (layer "F.Cu") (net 9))
 (segment (start 126.991467 99.109511) (end 127.325489 98.775489) (width 0.25) (layer "F.Cu") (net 9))
 (segment (start 127.775 103.125) (end 128.105 103.125) (width 0.25) (layer "F.Cu") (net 9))
 (segment (start 124.1605 94.65) (end 120.3505 98.46) (width 0.25) (layer "F.Cu") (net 9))
 (segment (start 136.682 97.380022) (end 136.682 97.025) (width 0.25) (layer "F.Cu") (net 9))
 (segment (start 133.6 97.3) (end 134.25 97.95) (width 0.25) (layer "F.Cu") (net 9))
 (segment (start 127.325489 98.775489) (end 128.05 98.775489) (width 0.25) (layer "F.Cu") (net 9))
 (segment (start 136.112022 97.95) (end 136.682 97.380022) (width 0.25) (layer "F.Cu") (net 9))
 (segment (start 120.562511 99.109511) (end 126.991467 99.109511) (width 0.25) (layer "F.Cu") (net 9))
 (segment (start 132.732 99.575) (end 133.6 98.707) (width 0.25) (layer "F.Cu") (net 9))
 (segment (start 129.235 101.995) (end 130.667022 101.995) (width 0.25) (layer "F.Cu") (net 9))
 (via (at 127.775 103.125) (size 0.8) (drill 0.4) (layers "F.Cu" "B.Cu") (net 9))
 (via (at 128.85 98.5745) (size 0.8) (drill 0.4) (layers "F.Cu" "B.Cu") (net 9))
 (segment (start 128.85 102.05) (end 127.775 103.125) (width 0.25) (layer "B.Cu") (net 9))
 (segment (start 128.85 98.5745) (end 128.85 102.05) (width 0.25) (layer "B.Cu") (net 9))
 (segment (start 129.150103 97.849989) (end 129.574511 98.274397) (width 0.25) (layer "F.Cu") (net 4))
 (segment (start 128.774511 99.299011) (end 128.774511 99.924991) (width 0.25) (layer "F.Cu") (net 4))
 (segment (start 119.913 94.65) (end 120.562511 94.000489) (width 0.25) (layer "F.Cu") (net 4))
 (segment (start 129.574511 98.274397) (end 129.574511 98.874603) (width 0.25) (layer "F.Cu") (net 4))
 (segment (start 126.424011 94.000489) (end 126.424011 97.849989) (width 0.25) (layer "F.Cu") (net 4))
 (segment (start 129.150103 99.299011) (end 128.774511 99.299011) (width 0.25) (layer "F.Cu") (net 4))
 (segment (start 128.774511 99.924991) (end 129.30001 99.924991) (width 0.25) (layer "F.Cu") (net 4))
 (segment (start 129.574511 98.874603) (end 129.150103 99.299011) (width 0.25) (layer "F.Cu") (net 4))
 (segment (start 129.30001 99.924991) (end 129.65 99.575) (width 0.25) (layer "F.Cu") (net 4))
 (segment (start 120.562511 94.000489) (end 126.424011 94.000489) (width 0.25) (layer "F.Cu") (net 4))
 (segment (start 126.424011 97.849989) (end 129.150103 97.849989) (width 0.25) (layer "F.Cu") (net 4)))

